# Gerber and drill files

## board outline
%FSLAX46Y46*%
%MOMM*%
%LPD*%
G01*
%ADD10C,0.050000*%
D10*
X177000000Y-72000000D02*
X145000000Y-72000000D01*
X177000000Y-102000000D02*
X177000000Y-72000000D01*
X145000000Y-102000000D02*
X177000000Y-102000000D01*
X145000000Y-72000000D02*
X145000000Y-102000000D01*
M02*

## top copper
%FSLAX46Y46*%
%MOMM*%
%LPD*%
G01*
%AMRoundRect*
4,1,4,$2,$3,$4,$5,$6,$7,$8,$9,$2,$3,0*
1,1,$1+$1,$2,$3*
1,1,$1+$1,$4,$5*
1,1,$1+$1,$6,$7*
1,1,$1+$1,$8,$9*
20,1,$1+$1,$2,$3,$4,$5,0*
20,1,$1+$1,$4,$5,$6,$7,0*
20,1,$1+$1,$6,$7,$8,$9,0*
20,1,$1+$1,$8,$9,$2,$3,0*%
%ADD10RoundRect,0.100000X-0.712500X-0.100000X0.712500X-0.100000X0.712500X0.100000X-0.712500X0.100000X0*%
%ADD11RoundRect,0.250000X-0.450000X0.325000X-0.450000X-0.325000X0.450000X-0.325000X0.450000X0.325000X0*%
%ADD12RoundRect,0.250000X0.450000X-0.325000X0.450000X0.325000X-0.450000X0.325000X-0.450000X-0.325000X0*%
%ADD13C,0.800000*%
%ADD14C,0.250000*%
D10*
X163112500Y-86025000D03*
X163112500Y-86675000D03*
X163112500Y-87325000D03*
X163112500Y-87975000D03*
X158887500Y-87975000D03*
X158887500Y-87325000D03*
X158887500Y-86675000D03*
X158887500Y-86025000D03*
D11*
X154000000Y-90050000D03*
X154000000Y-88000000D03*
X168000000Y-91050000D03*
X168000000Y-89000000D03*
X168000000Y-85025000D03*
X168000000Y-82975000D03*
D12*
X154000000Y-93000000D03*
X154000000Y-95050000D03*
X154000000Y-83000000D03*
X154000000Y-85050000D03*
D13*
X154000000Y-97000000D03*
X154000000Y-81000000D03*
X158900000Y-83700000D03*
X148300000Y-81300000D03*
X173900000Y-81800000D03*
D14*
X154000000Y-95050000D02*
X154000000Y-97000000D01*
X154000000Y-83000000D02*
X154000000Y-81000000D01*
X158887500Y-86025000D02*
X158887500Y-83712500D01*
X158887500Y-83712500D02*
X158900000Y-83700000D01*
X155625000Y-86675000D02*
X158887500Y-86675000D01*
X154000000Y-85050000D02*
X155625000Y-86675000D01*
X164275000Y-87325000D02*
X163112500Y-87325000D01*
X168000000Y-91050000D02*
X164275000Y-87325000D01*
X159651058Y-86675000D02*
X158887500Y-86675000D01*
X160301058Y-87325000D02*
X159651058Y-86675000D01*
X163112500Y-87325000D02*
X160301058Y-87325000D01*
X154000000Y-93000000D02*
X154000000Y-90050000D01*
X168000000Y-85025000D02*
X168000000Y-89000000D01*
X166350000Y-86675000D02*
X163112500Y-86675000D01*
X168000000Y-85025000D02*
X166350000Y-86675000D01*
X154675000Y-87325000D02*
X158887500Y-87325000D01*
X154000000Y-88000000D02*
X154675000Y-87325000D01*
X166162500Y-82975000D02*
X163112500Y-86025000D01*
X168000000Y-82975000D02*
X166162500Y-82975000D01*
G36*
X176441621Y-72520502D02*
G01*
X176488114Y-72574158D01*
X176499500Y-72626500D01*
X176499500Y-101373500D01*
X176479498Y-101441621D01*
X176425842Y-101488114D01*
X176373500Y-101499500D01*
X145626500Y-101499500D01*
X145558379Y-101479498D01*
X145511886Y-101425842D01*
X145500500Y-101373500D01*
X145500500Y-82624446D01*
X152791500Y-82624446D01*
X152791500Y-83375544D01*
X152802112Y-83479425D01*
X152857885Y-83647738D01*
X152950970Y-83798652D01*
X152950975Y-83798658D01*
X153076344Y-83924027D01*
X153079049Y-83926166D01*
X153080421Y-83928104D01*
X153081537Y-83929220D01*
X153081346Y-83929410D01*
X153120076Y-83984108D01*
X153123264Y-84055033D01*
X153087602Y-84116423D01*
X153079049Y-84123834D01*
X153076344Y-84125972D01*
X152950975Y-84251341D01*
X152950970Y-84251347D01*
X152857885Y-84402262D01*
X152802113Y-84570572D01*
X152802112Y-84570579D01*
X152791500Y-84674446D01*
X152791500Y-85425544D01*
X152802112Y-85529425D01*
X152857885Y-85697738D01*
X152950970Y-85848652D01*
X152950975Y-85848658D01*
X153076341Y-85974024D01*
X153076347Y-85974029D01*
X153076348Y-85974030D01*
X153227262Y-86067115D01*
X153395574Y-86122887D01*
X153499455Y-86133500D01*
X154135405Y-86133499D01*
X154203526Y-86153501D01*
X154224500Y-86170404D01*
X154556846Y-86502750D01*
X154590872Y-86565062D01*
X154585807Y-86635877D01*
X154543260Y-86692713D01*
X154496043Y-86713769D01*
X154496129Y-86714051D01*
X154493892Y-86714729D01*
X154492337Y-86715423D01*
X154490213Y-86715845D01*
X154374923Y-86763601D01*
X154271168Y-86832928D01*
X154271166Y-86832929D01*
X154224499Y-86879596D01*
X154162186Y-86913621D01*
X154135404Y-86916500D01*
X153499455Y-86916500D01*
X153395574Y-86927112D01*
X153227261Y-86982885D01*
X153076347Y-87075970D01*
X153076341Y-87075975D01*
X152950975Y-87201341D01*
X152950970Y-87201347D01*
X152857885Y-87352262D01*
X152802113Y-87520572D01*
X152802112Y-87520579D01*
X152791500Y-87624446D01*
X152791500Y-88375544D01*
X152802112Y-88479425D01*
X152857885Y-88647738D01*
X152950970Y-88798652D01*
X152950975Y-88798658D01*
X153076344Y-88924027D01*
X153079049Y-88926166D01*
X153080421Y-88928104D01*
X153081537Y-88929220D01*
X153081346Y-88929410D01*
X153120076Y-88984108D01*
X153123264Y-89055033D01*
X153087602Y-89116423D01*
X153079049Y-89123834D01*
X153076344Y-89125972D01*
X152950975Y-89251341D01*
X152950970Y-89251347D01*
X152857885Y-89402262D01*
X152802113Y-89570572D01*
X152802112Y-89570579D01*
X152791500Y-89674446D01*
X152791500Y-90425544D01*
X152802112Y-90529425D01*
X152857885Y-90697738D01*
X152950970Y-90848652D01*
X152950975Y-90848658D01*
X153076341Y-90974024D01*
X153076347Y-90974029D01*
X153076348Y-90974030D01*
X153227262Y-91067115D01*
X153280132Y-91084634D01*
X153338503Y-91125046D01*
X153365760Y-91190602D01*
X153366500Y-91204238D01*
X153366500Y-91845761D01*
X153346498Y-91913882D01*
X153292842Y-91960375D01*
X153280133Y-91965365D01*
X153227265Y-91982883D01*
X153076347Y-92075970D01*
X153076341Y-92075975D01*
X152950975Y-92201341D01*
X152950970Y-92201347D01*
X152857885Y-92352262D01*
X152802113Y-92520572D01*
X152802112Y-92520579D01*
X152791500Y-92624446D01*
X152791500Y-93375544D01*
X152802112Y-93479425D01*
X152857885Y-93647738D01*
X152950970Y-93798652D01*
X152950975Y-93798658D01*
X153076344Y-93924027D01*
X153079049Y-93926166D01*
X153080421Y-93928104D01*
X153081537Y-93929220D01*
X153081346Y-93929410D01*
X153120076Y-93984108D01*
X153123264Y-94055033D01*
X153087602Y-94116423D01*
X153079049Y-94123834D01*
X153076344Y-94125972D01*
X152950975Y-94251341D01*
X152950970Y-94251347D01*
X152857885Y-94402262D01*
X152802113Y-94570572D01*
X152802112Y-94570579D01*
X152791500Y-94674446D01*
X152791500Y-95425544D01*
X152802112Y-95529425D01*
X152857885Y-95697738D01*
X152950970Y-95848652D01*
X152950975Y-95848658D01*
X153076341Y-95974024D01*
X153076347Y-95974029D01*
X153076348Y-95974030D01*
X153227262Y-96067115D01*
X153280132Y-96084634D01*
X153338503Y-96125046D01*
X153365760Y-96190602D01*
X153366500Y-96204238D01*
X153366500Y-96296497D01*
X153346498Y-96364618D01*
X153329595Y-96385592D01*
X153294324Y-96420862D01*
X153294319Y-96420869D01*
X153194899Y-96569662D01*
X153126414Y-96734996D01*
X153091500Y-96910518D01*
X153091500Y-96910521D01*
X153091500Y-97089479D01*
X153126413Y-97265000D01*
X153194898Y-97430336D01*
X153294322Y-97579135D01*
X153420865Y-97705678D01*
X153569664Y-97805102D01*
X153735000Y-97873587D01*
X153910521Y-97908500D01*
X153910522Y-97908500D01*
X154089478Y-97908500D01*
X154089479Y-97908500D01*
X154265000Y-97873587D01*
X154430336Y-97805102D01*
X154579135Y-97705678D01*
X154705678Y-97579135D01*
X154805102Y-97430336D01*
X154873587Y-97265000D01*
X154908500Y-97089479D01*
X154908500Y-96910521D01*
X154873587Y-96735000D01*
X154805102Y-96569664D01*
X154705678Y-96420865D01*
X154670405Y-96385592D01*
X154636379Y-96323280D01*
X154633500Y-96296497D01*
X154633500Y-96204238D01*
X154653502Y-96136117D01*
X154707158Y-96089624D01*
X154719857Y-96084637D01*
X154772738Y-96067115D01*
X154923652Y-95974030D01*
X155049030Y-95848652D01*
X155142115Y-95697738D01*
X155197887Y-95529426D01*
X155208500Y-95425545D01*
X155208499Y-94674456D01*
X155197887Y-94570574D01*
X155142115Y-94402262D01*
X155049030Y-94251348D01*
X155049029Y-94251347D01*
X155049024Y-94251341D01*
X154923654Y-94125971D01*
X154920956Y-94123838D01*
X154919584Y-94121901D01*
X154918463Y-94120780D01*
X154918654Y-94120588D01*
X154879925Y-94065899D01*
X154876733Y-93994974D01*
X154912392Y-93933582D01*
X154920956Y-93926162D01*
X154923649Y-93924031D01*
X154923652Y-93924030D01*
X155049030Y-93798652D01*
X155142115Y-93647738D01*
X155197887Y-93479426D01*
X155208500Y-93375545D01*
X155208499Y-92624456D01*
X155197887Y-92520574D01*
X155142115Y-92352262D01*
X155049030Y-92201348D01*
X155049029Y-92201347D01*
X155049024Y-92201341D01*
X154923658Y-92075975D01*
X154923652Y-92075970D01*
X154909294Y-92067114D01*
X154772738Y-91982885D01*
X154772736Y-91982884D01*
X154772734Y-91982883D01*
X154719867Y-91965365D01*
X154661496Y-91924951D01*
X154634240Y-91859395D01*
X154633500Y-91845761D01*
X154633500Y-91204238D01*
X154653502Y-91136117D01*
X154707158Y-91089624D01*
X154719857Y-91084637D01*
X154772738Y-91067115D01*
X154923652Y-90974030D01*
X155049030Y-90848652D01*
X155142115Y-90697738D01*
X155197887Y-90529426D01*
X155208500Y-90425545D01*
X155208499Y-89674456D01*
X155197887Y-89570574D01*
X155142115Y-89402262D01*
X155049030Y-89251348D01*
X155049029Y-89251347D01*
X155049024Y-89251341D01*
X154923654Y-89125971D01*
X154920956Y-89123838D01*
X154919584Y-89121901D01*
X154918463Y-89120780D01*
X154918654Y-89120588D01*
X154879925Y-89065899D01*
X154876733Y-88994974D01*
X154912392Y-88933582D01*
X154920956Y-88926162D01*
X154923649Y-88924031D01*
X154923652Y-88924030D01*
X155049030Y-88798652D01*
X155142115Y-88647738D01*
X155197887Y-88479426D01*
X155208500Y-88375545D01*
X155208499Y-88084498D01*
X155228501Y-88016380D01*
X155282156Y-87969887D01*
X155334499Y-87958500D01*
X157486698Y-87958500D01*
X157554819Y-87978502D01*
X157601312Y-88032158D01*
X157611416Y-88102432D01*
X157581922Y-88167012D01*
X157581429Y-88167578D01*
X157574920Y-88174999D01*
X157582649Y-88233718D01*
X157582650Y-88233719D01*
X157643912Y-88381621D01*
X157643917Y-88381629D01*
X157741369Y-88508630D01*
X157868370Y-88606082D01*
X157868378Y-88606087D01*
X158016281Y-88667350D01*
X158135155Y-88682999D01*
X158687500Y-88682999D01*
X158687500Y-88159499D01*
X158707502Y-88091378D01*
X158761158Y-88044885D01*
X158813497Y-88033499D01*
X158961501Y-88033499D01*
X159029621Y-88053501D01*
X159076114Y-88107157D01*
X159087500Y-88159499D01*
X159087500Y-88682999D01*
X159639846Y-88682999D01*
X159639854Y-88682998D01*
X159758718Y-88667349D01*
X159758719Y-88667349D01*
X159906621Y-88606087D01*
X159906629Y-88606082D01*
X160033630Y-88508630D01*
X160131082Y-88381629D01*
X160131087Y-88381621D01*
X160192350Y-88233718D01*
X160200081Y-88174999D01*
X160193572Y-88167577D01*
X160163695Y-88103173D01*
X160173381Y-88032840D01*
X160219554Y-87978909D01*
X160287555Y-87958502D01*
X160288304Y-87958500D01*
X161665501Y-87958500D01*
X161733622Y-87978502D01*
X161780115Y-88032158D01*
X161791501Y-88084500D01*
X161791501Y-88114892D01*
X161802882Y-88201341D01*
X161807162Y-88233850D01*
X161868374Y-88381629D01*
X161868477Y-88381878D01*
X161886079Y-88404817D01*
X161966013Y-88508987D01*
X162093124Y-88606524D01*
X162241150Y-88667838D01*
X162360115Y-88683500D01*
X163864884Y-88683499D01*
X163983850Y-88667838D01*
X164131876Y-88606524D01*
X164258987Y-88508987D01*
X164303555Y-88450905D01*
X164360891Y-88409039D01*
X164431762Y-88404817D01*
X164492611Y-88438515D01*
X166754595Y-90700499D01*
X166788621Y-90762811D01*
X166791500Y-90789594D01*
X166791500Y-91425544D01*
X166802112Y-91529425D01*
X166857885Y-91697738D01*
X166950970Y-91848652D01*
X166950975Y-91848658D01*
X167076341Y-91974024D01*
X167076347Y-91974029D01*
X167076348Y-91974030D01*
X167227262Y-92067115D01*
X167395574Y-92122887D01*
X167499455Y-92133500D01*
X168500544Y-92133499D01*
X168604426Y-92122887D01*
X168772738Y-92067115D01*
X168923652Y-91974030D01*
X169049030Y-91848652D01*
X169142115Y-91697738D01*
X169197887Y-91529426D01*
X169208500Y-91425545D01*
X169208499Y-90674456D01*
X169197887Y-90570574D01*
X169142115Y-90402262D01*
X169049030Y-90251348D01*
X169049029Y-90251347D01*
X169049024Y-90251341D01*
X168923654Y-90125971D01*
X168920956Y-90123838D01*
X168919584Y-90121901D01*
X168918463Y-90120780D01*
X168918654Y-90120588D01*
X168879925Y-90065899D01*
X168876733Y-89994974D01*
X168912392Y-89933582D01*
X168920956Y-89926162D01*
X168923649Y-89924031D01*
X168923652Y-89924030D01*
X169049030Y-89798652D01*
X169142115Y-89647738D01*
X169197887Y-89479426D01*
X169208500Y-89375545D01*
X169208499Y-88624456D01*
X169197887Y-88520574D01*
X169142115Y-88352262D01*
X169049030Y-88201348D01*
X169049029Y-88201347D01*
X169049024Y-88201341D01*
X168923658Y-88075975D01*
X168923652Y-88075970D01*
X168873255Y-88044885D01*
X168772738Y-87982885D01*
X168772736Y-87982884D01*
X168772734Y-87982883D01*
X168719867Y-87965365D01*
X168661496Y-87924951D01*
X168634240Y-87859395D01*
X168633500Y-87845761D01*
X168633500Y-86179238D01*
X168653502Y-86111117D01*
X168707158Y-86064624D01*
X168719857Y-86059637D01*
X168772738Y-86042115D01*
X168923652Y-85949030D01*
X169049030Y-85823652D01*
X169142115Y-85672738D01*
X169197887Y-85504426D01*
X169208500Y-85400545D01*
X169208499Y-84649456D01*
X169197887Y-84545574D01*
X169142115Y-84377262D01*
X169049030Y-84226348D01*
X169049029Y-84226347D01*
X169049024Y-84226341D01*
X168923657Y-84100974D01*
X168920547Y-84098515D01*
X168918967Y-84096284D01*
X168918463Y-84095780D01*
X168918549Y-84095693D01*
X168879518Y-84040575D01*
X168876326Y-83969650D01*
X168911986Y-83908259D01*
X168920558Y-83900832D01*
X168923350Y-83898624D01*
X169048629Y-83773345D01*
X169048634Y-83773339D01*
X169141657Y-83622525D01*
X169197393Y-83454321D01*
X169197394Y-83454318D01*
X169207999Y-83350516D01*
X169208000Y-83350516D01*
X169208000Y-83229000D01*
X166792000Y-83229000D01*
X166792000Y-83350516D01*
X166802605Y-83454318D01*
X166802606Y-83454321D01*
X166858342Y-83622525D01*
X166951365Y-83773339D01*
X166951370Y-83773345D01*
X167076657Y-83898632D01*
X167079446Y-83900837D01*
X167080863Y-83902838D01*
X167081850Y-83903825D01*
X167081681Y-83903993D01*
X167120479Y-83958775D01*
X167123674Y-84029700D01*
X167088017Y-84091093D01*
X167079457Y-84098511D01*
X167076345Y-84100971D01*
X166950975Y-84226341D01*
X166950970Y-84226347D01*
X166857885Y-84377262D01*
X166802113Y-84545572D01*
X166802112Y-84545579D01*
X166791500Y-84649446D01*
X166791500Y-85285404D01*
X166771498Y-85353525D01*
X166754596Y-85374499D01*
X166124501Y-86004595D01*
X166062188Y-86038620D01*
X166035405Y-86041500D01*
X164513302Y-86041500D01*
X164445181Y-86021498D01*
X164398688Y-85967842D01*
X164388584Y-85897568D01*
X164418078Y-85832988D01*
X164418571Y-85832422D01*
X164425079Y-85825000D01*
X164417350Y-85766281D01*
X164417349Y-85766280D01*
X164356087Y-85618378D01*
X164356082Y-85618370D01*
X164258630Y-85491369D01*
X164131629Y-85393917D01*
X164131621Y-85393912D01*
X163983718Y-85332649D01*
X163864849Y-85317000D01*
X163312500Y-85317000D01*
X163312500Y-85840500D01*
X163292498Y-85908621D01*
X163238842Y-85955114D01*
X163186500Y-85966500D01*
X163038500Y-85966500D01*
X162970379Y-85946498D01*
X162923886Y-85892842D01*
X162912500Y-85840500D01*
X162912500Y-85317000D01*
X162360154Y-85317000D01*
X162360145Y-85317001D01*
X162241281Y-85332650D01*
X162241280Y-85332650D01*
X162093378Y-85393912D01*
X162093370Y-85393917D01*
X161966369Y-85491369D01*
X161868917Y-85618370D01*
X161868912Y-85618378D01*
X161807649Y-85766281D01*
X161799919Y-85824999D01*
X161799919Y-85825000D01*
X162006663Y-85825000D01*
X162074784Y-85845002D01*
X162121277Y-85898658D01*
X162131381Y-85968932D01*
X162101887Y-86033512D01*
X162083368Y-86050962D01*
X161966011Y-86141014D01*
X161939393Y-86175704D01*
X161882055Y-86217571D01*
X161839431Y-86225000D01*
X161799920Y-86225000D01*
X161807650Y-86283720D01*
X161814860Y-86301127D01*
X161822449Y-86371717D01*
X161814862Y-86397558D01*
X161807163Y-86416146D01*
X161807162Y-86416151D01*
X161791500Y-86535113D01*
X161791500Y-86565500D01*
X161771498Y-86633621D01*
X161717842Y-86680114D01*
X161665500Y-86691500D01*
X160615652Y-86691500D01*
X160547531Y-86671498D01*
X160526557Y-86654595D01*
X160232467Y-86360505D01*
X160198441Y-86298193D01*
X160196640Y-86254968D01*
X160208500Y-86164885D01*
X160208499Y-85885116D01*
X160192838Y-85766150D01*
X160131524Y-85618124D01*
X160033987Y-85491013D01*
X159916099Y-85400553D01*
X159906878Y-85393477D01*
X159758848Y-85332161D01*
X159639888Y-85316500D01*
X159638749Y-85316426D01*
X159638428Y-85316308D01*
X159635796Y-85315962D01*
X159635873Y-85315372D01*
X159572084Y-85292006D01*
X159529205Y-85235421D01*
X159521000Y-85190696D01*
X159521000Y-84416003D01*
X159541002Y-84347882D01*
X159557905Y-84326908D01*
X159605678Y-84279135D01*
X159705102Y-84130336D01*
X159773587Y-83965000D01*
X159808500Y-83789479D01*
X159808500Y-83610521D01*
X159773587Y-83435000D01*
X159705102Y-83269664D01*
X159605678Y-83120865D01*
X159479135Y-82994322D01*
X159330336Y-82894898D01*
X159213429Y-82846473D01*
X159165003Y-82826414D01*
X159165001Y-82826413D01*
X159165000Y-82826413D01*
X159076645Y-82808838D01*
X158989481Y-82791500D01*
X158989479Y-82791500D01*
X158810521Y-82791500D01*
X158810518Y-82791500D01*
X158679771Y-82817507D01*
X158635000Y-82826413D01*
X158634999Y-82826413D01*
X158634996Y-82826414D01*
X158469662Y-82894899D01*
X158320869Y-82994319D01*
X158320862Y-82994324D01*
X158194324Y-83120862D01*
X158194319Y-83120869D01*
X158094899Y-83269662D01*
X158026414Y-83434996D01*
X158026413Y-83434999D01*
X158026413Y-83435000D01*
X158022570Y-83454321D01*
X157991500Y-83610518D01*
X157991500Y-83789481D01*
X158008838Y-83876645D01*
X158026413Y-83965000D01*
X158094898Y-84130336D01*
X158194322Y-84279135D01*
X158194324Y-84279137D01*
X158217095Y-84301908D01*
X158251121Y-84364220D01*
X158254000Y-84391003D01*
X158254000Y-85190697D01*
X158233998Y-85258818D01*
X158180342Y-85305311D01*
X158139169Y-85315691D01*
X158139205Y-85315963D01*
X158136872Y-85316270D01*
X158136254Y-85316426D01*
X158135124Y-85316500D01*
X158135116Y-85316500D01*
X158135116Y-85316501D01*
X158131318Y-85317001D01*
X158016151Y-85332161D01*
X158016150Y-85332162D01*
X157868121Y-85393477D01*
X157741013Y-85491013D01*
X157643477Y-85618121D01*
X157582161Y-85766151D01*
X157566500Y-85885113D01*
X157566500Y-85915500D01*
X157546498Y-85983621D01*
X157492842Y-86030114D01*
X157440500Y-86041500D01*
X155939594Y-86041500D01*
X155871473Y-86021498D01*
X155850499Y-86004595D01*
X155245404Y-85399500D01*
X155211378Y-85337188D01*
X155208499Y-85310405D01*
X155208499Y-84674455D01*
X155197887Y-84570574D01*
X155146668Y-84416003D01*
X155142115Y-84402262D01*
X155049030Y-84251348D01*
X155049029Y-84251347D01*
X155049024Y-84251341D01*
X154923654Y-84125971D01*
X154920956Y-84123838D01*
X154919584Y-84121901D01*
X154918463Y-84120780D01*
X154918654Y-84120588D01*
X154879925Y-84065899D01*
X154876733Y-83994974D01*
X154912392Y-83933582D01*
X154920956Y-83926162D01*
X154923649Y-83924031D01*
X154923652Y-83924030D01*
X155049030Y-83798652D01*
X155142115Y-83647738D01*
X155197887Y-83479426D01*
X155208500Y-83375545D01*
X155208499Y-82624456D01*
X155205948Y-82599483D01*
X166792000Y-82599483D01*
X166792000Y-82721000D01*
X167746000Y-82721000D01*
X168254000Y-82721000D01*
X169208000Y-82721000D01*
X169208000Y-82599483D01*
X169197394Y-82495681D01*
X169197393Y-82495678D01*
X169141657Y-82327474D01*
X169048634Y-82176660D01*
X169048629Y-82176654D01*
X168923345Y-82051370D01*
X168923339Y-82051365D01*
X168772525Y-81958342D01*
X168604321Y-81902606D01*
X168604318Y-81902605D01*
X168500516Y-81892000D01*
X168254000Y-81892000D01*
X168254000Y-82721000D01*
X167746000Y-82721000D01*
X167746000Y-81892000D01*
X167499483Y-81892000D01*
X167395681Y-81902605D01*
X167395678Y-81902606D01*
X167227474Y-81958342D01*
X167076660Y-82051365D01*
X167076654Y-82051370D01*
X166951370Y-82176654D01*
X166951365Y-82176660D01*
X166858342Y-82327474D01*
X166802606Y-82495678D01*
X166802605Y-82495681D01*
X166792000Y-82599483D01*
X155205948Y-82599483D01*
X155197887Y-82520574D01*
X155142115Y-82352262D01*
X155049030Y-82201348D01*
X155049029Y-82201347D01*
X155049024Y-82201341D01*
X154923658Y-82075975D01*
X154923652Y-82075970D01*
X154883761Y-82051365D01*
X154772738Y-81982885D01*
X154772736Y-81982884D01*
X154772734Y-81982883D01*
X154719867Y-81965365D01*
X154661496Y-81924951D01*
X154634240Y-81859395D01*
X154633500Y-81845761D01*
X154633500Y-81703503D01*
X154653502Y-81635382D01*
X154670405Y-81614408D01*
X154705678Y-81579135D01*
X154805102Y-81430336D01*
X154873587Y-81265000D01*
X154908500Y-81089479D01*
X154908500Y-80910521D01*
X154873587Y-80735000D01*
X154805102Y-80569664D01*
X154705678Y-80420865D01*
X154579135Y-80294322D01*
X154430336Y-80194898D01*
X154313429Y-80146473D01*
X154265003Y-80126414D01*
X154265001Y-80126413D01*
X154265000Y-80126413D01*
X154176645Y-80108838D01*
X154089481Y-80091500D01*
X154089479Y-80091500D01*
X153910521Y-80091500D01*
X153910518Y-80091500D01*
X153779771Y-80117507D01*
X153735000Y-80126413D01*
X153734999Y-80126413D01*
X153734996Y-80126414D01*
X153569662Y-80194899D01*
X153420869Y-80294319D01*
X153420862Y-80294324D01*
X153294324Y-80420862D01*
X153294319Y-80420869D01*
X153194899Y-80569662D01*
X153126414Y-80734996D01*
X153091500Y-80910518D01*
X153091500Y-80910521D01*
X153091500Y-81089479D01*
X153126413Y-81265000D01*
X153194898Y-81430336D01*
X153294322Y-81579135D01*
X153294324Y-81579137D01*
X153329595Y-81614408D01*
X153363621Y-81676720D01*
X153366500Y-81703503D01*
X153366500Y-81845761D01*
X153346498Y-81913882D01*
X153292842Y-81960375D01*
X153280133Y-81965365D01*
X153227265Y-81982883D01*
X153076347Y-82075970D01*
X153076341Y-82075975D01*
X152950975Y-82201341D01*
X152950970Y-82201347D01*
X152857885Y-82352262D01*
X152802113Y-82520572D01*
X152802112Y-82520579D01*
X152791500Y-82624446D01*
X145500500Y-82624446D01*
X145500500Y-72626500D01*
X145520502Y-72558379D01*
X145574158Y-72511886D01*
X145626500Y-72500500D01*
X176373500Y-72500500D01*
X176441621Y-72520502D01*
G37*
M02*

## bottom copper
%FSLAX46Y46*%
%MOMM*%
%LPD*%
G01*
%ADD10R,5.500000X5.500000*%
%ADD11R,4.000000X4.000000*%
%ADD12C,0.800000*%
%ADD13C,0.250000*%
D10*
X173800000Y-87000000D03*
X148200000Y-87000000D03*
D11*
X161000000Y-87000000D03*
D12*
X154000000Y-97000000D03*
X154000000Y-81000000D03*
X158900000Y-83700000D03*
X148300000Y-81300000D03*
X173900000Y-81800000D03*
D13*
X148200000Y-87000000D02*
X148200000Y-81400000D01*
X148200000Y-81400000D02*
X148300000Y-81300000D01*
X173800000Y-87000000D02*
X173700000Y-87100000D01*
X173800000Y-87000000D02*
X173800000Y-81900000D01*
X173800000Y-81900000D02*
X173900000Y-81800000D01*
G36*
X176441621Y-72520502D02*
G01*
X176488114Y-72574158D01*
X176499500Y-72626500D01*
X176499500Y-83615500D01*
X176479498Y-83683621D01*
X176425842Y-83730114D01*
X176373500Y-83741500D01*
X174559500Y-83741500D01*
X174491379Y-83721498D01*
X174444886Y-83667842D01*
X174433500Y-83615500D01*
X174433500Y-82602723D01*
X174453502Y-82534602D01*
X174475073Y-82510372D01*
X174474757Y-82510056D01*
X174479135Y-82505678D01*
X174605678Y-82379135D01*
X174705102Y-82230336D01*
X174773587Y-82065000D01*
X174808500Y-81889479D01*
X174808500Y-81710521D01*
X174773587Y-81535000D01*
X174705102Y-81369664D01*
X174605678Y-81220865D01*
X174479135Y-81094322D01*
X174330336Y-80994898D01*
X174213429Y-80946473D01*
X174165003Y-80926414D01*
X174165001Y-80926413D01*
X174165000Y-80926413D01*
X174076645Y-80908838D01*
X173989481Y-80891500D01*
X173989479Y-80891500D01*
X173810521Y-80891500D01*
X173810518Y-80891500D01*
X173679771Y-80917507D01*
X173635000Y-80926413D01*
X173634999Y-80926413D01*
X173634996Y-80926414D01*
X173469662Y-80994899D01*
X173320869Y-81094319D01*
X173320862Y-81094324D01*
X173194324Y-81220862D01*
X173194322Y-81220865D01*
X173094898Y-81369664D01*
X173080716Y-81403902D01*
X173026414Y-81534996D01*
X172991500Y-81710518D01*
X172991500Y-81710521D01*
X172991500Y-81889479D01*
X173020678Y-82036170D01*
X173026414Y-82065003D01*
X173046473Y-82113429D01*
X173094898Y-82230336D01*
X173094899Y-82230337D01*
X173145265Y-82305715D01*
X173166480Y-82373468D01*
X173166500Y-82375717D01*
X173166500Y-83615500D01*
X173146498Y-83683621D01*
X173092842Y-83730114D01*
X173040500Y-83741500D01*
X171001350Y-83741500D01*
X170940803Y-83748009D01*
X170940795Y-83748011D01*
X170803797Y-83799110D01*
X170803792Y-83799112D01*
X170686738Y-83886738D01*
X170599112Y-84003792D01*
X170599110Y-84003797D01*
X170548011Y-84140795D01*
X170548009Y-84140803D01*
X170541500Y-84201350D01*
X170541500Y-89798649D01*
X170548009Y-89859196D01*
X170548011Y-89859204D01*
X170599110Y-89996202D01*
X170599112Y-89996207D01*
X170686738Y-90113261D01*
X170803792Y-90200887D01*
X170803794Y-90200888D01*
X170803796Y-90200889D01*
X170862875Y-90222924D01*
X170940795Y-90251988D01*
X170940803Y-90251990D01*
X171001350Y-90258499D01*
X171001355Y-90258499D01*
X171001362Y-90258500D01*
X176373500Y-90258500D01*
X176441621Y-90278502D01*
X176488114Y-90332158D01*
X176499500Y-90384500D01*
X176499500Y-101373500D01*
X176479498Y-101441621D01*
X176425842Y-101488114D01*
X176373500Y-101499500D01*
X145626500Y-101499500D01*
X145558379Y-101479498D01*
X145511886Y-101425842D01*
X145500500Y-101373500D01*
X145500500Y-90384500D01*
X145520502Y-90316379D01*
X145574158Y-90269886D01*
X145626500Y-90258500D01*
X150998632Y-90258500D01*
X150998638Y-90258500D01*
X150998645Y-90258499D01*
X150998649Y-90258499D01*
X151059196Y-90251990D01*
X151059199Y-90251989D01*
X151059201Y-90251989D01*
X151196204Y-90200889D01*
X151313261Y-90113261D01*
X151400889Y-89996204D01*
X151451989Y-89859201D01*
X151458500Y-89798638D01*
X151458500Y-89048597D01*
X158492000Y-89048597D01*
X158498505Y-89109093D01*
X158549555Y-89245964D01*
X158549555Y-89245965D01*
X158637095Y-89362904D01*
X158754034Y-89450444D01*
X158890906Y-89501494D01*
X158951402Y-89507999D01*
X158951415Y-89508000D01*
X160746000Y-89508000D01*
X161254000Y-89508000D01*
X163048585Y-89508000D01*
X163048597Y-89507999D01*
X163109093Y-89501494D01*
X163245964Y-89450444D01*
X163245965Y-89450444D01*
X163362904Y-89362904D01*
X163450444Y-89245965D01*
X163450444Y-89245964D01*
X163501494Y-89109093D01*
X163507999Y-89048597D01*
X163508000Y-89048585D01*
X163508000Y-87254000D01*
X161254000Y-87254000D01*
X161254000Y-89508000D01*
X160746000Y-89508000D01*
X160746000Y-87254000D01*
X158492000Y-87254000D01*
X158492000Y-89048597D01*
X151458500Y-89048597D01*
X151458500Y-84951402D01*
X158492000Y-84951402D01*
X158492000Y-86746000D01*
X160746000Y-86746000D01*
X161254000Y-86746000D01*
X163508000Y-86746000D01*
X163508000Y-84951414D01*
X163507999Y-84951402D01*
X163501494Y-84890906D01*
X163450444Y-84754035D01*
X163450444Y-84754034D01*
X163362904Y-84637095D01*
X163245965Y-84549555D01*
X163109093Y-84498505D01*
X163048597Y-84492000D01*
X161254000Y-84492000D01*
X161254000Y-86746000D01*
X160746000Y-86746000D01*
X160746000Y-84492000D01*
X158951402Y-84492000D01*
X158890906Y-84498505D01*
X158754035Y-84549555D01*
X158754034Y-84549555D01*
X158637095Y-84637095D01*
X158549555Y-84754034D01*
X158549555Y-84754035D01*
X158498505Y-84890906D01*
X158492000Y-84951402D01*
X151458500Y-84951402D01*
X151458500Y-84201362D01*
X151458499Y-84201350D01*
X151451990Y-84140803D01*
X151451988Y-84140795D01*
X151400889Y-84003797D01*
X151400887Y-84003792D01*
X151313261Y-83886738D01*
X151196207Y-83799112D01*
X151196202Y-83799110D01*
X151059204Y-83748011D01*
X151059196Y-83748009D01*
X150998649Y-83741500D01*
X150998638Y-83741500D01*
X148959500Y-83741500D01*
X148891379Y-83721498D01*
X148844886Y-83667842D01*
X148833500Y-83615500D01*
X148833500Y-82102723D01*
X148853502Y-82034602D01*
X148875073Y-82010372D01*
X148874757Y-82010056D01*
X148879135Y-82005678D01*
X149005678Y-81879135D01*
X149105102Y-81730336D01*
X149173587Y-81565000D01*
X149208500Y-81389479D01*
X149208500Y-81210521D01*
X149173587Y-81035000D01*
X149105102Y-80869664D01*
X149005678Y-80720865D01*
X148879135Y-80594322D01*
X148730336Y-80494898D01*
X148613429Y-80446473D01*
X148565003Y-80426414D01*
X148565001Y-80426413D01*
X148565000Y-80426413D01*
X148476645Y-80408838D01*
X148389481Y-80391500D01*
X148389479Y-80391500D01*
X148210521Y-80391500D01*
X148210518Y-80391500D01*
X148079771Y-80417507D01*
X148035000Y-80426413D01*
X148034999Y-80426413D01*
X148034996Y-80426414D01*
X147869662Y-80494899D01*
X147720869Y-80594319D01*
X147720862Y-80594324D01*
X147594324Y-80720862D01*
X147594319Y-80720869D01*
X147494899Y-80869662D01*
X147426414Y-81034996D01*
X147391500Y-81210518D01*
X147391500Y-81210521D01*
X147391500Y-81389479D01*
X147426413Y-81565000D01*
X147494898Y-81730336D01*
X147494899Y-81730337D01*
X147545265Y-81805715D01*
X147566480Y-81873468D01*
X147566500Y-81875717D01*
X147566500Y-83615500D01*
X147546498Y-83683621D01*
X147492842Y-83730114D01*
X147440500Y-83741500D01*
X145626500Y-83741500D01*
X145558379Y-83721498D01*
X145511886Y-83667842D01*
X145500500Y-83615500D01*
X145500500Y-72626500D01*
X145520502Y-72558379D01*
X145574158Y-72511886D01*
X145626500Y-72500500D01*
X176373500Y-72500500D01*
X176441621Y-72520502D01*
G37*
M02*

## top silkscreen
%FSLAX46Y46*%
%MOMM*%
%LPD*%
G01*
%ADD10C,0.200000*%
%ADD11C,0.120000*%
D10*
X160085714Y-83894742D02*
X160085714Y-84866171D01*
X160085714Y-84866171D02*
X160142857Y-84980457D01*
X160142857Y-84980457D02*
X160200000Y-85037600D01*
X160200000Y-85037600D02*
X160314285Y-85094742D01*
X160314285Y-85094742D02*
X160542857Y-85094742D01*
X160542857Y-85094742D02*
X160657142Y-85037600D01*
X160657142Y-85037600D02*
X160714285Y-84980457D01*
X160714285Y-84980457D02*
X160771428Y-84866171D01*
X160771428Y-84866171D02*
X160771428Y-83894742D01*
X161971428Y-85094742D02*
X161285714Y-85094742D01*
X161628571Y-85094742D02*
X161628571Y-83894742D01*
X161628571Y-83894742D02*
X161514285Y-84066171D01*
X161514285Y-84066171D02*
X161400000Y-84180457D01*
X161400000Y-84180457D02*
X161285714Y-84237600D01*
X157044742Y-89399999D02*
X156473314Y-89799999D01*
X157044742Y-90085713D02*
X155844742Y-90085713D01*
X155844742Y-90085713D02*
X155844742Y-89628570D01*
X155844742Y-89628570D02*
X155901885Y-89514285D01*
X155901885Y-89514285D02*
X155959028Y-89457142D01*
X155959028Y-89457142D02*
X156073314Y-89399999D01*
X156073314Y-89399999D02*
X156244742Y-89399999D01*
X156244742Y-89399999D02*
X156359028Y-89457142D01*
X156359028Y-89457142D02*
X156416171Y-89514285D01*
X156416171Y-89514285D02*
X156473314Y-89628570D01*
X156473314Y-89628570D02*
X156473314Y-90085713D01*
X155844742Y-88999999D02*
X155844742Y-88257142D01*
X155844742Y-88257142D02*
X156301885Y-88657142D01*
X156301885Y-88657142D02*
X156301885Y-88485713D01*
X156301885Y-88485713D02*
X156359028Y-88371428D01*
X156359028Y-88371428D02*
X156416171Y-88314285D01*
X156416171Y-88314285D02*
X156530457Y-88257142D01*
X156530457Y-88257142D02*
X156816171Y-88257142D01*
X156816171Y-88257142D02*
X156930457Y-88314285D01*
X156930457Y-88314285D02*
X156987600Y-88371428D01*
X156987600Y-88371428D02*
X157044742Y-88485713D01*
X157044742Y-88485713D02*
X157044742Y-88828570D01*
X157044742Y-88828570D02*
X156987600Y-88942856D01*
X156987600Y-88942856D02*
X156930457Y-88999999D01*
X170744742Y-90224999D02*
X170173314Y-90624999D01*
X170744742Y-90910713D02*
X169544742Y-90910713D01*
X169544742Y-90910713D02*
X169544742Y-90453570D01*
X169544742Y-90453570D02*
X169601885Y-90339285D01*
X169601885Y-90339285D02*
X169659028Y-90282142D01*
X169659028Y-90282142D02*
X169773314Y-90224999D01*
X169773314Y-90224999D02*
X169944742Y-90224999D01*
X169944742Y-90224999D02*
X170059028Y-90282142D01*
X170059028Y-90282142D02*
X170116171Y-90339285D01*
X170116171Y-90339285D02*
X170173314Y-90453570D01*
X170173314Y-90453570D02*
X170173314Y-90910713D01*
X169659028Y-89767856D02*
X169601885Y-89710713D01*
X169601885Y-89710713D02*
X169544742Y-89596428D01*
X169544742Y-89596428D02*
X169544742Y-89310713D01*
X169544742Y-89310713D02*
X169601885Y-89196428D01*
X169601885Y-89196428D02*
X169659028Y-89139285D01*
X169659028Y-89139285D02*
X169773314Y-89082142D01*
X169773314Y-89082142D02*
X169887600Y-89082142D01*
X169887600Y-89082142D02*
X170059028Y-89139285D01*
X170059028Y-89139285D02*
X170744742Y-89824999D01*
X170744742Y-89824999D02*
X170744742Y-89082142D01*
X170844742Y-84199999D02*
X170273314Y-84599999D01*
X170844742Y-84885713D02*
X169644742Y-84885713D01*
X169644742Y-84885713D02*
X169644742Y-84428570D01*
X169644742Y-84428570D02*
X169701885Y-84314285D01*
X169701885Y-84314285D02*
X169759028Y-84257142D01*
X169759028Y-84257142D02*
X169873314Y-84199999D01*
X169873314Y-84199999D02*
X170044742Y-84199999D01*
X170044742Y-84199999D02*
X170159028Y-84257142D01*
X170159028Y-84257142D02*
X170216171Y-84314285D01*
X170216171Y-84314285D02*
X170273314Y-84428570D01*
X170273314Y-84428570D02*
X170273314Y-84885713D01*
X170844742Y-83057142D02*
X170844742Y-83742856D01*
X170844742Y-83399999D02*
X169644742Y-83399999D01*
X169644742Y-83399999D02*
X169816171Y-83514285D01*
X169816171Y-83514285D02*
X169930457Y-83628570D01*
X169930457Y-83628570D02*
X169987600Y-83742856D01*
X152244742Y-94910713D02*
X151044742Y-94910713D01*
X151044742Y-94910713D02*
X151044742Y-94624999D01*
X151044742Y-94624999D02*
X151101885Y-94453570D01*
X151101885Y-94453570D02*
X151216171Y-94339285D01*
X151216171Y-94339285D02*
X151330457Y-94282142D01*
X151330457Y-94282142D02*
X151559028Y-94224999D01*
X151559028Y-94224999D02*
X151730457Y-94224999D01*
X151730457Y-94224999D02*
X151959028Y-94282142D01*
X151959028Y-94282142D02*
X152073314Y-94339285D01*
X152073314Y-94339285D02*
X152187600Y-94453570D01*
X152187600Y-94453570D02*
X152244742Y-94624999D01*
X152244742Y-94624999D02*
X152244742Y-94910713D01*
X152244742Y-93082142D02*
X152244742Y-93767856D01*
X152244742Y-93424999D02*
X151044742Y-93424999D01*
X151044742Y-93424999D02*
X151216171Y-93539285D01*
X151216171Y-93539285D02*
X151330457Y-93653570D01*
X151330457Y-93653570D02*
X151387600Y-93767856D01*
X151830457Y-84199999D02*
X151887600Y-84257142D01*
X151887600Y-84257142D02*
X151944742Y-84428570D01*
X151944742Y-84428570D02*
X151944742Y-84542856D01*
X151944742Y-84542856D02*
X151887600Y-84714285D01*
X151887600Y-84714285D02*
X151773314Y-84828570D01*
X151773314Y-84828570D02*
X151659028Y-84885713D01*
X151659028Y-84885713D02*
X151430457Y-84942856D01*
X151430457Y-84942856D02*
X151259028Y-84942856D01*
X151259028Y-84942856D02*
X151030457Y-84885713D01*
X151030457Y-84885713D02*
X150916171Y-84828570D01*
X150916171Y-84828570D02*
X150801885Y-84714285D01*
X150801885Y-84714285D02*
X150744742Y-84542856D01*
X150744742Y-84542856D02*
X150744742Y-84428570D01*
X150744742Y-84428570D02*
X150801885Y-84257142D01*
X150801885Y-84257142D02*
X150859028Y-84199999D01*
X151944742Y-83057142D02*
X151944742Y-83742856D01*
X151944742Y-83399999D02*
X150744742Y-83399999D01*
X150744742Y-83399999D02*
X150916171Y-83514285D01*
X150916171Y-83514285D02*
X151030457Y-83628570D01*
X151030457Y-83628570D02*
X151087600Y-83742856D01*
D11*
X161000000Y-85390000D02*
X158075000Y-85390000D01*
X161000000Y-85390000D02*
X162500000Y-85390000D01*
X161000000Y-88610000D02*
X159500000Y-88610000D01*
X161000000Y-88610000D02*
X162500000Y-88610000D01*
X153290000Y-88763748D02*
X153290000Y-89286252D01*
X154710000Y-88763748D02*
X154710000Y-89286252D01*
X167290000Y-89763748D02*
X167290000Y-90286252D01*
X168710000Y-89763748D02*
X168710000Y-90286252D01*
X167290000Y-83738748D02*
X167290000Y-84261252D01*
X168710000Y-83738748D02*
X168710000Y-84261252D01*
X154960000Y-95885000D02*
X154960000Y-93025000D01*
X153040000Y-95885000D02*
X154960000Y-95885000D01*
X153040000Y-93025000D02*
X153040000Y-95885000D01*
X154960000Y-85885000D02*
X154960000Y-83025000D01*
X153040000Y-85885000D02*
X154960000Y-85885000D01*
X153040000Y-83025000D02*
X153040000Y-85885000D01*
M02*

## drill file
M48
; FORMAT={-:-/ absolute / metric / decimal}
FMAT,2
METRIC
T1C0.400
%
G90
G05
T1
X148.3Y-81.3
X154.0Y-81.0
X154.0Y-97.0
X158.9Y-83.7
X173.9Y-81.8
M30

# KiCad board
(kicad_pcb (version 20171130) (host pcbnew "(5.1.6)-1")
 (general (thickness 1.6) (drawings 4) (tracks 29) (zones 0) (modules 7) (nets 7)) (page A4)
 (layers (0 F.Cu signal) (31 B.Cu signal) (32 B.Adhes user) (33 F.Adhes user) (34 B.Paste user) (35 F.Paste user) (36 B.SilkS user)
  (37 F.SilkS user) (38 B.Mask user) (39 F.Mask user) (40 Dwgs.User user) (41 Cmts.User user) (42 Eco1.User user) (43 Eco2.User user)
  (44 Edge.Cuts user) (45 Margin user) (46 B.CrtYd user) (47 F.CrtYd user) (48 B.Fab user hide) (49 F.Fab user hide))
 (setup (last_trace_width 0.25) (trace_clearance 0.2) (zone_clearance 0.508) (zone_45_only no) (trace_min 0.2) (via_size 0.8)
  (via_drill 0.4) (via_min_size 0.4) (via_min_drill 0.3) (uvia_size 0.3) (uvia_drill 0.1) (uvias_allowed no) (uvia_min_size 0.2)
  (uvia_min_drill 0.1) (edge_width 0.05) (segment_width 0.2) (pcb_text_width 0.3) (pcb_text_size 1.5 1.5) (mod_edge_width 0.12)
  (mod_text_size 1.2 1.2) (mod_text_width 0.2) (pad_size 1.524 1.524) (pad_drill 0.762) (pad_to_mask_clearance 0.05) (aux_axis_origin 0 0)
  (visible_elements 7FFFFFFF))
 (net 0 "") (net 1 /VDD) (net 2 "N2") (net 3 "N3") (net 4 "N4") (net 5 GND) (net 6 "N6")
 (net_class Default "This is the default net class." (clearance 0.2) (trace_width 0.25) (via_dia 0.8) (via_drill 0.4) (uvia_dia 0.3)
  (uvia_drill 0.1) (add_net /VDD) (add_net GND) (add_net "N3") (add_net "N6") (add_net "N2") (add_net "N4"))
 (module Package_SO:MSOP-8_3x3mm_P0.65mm (layer F.Cu) (at 161 87)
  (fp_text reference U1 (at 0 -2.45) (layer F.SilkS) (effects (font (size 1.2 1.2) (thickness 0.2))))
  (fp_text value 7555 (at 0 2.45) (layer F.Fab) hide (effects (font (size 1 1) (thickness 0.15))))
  (fp_line (start 0 -1.61) (end -2.925 -1.61) (layer F.SilkS) (width 0.12))
  (fp_line (start 0 -1.61) (end 1.5 -1.61) (layer F.SilkS) (width 0.12))
  (fp_line (start 0 1.61) (end -1.5 1.61) (layer F.SilkS) (width 0.12))
  (fp_line (start 0 1.61) (end 1.5 1.61) (layer F.SilkS) (width 0.12))
  (pad 8 smd roundrect (at 2.1125 -0.975) (size 1.625 0.4) (layers F.Cu F.Paste F.Mask) (roundrect_rratio 0.25) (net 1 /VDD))
  (pad 7 smd roundrect (at 2.1125 -0.325) (size 1.625 0.4) (layers F.Cu F.Paste F.Mask) (roundrect_rratio 0.25) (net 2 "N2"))
  (pad 6 smd roundrect (at 2.1125 0.325) (size 1.625 0.4) (layers F.Cu F.Paste F.Mask) (roundrect_rratio 0.25) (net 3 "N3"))
  (pad 5 smd roundrect (at 2.1125 0.975) (size 1.625 0.4) (layers F.Cu F.Paste F.Mask) (roundrect_rratio 0.25))
  (pad 4 smd roundrect (at -2.1125 0.975) (size 1.625 0.4) (layers F.Cu F.Paste F.Mask) (roundrect_rratio 0.25) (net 1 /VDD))
  (pad 3 smd roundrect (at -2.1125 0.325) (size 1.625 0.4) (layers F.Cu F.Paste F.Mask) (roundrect_rratio 0.25) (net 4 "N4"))
  (pad 2 smd roundrect (at -2.1125 -0.325) (size 1.625 0.4) (layers F.Cu F.Paste F.Mask) (roundrect_rratio 0.25) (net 3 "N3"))
  (pad 1 smd roundrect (at -2.1125 -0.975) (size 1.625 0.4) (layers F.Cu F.Paste F.Mask) (roundrect_rratio 0.25) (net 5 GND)))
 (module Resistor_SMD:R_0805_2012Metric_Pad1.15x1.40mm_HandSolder (layer F.Cu) (at 154 89.025 270)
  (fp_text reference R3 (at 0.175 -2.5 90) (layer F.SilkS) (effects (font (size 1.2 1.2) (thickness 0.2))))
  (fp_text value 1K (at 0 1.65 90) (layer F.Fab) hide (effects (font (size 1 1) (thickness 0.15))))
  (fp_line (start -0.261252 0.71) (end 0.261252 0.71) (layer F.SilkS) (width 0.12))
  (fp_line (start -0.261252 -0.71) (end 0.261252 -0.71) (layer F.SilkS) (width 0.12))
  (pad 2 smd roundrect (at 1.025 0 270) (size 1.15 1.4) (layers F.Cu F.Paste F.Mask) (roundrect_rratio 0.217391) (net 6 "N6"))
  (pad 1 smd roundrect (at -1.025 0 270) (size 1.15 1.4) (layers F.Cu F.Paste F.Mask) (roundrect_rratio 0.217391) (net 4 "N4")))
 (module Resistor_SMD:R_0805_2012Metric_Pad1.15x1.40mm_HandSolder (layer F.Cu) (at 168 90.025 270)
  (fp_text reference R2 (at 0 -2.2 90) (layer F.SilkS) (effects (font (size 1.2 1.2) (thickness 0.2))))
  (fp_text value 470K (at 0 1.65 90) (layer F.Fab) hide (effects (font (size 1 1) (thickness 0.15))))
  (fp_line (start -0.261252 0.71) (end 0.261252 0.71) (layer F.SilkS) (width 0.12))
  (fp_line (start -0.261252 -0.71) (end 0.261252 -0.71) (layer F.SilkS) (width 0.12))
  (pad 2 smd roundrect (at 1.025 0 270) (size 1.15 1.4) (layers F.Cu F.Paste F.Mask) (roundrect_rratio 0.217391) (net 3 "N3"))
  (pad 1 smd roundrect (at -1.025 0 270) (size 1.15 1.4) (layers F.Cu F.Paste F.Mask) (roundrect_rratio 0.217391) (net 2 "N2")))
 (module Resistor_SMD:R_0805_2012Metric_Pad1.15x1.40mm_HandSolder (layer F.Cu) (at 168 84 270)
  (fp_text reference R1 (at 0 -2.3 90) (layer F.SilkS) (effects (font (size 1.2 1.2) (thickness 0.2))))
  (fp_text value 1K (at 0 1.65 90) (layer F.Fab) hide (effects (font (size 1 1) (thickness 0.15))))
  (fp_line (start -0.261252 0.71) (end 0.261252 0.71) (layer F.SilkS) (width 0.12))
  (fp_line (start -0.261252 -0.71) (end 0.261252 -0.71) (layer F.SilkS) (width 0.12))
  (pad 2 smd roundrect (at 1.025 0 270) (size 1.15 1.4) (layers F.Cu F.Paste F.Mask) (roundrect_rratio 0.217391) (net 2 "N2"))
  (pad 1 smd roundrect (at -1.025 0 270) (size 1.15 1.4) (layers F.Cu F.Paste F.Mask) (roundrect_rratio 0.217391) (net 1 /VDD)))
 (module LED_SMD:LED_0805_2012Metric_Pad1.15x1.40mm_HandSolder (layer F.Cu) (at 154 94.025 90)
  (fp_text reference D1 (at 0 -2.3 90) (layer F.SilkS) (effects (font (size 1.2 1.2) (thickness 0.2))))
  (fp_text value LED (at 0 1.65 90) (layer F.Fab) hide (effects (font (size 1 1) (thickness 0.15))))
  (fp_line (start -1.86 0.96) (end 1 0.96) (layer F.SilkS) (width 0.12))
  (fp_line (start -1.86 -0.96) (end -1.86 0.96) (layer F.SilkS) (width 0.12))
  (fp_line (start 1 -0.96) (end -1.86 -0.96) (layer F.SilkS) (width 0.12))
  (pad 2 smd roundrect (at 1.025 0 90) (size 1.15 1.4) (layers F.Cu F.Paste F.Mask) (roundrect_rratio 0.217391) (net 6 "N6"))
  (pad 1 smd roundrect (at -1.025 0 90) (size 1.15 1.4) (layers F.Cu F.Paste F.Mask) (roundrect_rratio 0.217391) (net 5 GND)))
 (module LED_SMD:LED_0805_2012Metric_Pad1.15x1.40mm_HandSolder (layer F.Cu) (at 154 84.025 90)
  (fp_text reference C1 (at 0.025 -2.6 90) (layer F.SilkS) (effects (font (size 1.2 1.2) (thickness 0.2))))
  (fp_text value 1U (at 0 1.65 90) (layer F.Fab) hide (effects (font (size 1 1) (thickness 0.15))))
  (fp_line (start -1.86 0.96) (end 1 0.96) (layer F.SilkS) (width 0.12))
  (fp_line (start -1.86 -0.96) (end -1.86 0.96) (layer F.SilkS) (width 0.12))
  (fp_line (start 1 -0.96) (end -1.86 -0.96) (layer F.SilkS) (width 0.12))
  (pad 2 smd roundrect (at 1.025 0 90) (size 1.15 1.4) (layers F.Cu F.Paste F.Mask) (roundrect_rratio 0.217391) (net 5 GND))
  (pad 1 smd roundrect (at -1.025 0 90) (size 1.15 1.4) (layers F.Cu F.Paste F.Mask) (roundrect_rratio 0.217391) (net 3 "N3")))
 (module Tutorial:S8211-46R (layer B.Cu) (at 161 87)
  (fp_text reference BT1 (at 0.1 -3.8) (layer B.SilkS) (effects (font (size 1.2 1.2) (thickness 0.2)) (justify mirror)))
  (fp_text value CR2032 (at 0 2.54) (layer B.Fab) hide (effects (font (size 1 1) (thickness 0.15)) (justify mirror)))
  (pad 1 smd rect (at 12.8 0) (size 5.5 5.5) (layers B.Cu B.Paste B.Mask) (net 1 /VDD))
  (pad 1 smd rect (at -12.8 0) (size 5.5 5.5) (layers B.Cu B.Paste B.Mask) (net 1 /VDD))
  (pad 2 smd rect (at 0 0) (size 4 4) (layers B.Cu B.Paste B.Mask) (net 5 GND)))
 (gr_line (start 177 72) (end 145 72) (layer Edge.Cuts) (width 0.05))
 (gr_line (start 177 102) (end 177 72) (layer Edge.Cuts) (width 0.05))
 (gr_line (start 145 102) (end 177 102) (layer Edge.Cuts) (width 0.05))
 (gr_line (start 145 72) (end 145 102) (layer Edge.Cuts) (width 0.05))
 (via (at 154 97) (size 0.8) (drill 0.4) (layers F.Cu B.Cu) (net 5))
 (segment (start 154 95.05) (end 154 97) (width 0.25) (layer F.Cu) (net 5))
 (via (at 154 81) (size 0.8) (drill 0.4) (layers F.Cu B.Cu) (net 5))
 (segment (start 154 83) (end 154 81) (width 0.25) (layer F.Cu) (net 5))
 (via (at 158.9 83.7) (size 0.8) (drill 0.4) (layers F.Cu B.Cu) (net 5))
 (segment (start 158.8875 86.025) (end 158.8875 83.7125) (width 0.25) (layer F.Cu) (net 5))
 (segment (start 158.8875 83.7125) (end 158.9 83.7) (width 0.25) (layer F.Cu) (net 5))
 (segment (start 155.625 86.675) (end 158.8875 86.675) (width 0.25) (layer F.Cu) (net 3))
 (segment (start 154 85.05) (end 155.625 86.675) (width 0.25) (layer F.Cu) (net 3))
 (segment (start 164.275 87.325) (end 163.1125 87.325) (width 0.25) (layer F.Cu) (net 3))
 (segment (start 168 91.05) (end 164.275 87.325) (width 0.25) (layer F.Cu) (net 3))
 (segment (start 159.651058 86.675) (end 158.8875 86.675) (width 0.25) (layer F.Cu) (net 3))
 (segment (start 160.301058 87.325) (end 159.651058 86.675) (width 0.25) (layer F.Cu) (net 3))
 (segment (start 163.1125 87.325) (end 160.301058 87.325) (width 0.25) (layer F.Cu) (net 3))
 (segment (start 154 93) (end 154 90.05) (width 0.25) (layer F.Cu) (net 6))
 (segment (start 168 85.025) (end 168 89) (width 0.25) (layer F.Cu) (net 2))
 (segment (start 166.35 86.675) (end 163.1125 86.675) (width 0.25) (layer F.Cu) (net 2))
 (segment (start 168 85.025) (end 166.35 86.675) (width 0.25) (layer F.Cu) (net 2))
 (segment (start 154.675 87.325) (end 158.8875 87.325) (width 0.25) (layer F.Cu) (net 4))
 (segment (start 154 88) (end 154.675 87.325) (width 0.25) (layer F.Cu) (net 4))
 (segment (start 166.1625 82.975) (end 163.1125 86.025) (width 0.25) (layer F.Cu) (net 1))
 (segment (start 168 82.975) (end 166.1625 82.975) (width 0.25) (layer F.Cu) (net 1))
 (segment (start 148.2 87) (end 148.2 81.4) (width 0.25) (layer B.Cu) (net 1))
 (via (at 148.3 81.3) (size 0.8) (drill 0.4) (layers F.Cu B.Cu) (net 1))
 (segment (start 148.2 81.4) (end 148.3 81.3) (width 0.25) (layer B.Cu) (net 1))
 (segment (start 173.8 87) (end 173.7 87.1) (width 0.25) (layer B.Cu) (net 1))
 (via (at 173.9 81.8) (size 0.8) (drill 0.4) (layers F.Cu B.Cu) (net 1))
 (segment (start 173.8 87) (end 173.8 81.9) (width 0.25) (layer B.Cu) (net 1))
 (segment (start 173.8 81.9) (end 173.9 81.8) (width 0.25) (layer B.Cu) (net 1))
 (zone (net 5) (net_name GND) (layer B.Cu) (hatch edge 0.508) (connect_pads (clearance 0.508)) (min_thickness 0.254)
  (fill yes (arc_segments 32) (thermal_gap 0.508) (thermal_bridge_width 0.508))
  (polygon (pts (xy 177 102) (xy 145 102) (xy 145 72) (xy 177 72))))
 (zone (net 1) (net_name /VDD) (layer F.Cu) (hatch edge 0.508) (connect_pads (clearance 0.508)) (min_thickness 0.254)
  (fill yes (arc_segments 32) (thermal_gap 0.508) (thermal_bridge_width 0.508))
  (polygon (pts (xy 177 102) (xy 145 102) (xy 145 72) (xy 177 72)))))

